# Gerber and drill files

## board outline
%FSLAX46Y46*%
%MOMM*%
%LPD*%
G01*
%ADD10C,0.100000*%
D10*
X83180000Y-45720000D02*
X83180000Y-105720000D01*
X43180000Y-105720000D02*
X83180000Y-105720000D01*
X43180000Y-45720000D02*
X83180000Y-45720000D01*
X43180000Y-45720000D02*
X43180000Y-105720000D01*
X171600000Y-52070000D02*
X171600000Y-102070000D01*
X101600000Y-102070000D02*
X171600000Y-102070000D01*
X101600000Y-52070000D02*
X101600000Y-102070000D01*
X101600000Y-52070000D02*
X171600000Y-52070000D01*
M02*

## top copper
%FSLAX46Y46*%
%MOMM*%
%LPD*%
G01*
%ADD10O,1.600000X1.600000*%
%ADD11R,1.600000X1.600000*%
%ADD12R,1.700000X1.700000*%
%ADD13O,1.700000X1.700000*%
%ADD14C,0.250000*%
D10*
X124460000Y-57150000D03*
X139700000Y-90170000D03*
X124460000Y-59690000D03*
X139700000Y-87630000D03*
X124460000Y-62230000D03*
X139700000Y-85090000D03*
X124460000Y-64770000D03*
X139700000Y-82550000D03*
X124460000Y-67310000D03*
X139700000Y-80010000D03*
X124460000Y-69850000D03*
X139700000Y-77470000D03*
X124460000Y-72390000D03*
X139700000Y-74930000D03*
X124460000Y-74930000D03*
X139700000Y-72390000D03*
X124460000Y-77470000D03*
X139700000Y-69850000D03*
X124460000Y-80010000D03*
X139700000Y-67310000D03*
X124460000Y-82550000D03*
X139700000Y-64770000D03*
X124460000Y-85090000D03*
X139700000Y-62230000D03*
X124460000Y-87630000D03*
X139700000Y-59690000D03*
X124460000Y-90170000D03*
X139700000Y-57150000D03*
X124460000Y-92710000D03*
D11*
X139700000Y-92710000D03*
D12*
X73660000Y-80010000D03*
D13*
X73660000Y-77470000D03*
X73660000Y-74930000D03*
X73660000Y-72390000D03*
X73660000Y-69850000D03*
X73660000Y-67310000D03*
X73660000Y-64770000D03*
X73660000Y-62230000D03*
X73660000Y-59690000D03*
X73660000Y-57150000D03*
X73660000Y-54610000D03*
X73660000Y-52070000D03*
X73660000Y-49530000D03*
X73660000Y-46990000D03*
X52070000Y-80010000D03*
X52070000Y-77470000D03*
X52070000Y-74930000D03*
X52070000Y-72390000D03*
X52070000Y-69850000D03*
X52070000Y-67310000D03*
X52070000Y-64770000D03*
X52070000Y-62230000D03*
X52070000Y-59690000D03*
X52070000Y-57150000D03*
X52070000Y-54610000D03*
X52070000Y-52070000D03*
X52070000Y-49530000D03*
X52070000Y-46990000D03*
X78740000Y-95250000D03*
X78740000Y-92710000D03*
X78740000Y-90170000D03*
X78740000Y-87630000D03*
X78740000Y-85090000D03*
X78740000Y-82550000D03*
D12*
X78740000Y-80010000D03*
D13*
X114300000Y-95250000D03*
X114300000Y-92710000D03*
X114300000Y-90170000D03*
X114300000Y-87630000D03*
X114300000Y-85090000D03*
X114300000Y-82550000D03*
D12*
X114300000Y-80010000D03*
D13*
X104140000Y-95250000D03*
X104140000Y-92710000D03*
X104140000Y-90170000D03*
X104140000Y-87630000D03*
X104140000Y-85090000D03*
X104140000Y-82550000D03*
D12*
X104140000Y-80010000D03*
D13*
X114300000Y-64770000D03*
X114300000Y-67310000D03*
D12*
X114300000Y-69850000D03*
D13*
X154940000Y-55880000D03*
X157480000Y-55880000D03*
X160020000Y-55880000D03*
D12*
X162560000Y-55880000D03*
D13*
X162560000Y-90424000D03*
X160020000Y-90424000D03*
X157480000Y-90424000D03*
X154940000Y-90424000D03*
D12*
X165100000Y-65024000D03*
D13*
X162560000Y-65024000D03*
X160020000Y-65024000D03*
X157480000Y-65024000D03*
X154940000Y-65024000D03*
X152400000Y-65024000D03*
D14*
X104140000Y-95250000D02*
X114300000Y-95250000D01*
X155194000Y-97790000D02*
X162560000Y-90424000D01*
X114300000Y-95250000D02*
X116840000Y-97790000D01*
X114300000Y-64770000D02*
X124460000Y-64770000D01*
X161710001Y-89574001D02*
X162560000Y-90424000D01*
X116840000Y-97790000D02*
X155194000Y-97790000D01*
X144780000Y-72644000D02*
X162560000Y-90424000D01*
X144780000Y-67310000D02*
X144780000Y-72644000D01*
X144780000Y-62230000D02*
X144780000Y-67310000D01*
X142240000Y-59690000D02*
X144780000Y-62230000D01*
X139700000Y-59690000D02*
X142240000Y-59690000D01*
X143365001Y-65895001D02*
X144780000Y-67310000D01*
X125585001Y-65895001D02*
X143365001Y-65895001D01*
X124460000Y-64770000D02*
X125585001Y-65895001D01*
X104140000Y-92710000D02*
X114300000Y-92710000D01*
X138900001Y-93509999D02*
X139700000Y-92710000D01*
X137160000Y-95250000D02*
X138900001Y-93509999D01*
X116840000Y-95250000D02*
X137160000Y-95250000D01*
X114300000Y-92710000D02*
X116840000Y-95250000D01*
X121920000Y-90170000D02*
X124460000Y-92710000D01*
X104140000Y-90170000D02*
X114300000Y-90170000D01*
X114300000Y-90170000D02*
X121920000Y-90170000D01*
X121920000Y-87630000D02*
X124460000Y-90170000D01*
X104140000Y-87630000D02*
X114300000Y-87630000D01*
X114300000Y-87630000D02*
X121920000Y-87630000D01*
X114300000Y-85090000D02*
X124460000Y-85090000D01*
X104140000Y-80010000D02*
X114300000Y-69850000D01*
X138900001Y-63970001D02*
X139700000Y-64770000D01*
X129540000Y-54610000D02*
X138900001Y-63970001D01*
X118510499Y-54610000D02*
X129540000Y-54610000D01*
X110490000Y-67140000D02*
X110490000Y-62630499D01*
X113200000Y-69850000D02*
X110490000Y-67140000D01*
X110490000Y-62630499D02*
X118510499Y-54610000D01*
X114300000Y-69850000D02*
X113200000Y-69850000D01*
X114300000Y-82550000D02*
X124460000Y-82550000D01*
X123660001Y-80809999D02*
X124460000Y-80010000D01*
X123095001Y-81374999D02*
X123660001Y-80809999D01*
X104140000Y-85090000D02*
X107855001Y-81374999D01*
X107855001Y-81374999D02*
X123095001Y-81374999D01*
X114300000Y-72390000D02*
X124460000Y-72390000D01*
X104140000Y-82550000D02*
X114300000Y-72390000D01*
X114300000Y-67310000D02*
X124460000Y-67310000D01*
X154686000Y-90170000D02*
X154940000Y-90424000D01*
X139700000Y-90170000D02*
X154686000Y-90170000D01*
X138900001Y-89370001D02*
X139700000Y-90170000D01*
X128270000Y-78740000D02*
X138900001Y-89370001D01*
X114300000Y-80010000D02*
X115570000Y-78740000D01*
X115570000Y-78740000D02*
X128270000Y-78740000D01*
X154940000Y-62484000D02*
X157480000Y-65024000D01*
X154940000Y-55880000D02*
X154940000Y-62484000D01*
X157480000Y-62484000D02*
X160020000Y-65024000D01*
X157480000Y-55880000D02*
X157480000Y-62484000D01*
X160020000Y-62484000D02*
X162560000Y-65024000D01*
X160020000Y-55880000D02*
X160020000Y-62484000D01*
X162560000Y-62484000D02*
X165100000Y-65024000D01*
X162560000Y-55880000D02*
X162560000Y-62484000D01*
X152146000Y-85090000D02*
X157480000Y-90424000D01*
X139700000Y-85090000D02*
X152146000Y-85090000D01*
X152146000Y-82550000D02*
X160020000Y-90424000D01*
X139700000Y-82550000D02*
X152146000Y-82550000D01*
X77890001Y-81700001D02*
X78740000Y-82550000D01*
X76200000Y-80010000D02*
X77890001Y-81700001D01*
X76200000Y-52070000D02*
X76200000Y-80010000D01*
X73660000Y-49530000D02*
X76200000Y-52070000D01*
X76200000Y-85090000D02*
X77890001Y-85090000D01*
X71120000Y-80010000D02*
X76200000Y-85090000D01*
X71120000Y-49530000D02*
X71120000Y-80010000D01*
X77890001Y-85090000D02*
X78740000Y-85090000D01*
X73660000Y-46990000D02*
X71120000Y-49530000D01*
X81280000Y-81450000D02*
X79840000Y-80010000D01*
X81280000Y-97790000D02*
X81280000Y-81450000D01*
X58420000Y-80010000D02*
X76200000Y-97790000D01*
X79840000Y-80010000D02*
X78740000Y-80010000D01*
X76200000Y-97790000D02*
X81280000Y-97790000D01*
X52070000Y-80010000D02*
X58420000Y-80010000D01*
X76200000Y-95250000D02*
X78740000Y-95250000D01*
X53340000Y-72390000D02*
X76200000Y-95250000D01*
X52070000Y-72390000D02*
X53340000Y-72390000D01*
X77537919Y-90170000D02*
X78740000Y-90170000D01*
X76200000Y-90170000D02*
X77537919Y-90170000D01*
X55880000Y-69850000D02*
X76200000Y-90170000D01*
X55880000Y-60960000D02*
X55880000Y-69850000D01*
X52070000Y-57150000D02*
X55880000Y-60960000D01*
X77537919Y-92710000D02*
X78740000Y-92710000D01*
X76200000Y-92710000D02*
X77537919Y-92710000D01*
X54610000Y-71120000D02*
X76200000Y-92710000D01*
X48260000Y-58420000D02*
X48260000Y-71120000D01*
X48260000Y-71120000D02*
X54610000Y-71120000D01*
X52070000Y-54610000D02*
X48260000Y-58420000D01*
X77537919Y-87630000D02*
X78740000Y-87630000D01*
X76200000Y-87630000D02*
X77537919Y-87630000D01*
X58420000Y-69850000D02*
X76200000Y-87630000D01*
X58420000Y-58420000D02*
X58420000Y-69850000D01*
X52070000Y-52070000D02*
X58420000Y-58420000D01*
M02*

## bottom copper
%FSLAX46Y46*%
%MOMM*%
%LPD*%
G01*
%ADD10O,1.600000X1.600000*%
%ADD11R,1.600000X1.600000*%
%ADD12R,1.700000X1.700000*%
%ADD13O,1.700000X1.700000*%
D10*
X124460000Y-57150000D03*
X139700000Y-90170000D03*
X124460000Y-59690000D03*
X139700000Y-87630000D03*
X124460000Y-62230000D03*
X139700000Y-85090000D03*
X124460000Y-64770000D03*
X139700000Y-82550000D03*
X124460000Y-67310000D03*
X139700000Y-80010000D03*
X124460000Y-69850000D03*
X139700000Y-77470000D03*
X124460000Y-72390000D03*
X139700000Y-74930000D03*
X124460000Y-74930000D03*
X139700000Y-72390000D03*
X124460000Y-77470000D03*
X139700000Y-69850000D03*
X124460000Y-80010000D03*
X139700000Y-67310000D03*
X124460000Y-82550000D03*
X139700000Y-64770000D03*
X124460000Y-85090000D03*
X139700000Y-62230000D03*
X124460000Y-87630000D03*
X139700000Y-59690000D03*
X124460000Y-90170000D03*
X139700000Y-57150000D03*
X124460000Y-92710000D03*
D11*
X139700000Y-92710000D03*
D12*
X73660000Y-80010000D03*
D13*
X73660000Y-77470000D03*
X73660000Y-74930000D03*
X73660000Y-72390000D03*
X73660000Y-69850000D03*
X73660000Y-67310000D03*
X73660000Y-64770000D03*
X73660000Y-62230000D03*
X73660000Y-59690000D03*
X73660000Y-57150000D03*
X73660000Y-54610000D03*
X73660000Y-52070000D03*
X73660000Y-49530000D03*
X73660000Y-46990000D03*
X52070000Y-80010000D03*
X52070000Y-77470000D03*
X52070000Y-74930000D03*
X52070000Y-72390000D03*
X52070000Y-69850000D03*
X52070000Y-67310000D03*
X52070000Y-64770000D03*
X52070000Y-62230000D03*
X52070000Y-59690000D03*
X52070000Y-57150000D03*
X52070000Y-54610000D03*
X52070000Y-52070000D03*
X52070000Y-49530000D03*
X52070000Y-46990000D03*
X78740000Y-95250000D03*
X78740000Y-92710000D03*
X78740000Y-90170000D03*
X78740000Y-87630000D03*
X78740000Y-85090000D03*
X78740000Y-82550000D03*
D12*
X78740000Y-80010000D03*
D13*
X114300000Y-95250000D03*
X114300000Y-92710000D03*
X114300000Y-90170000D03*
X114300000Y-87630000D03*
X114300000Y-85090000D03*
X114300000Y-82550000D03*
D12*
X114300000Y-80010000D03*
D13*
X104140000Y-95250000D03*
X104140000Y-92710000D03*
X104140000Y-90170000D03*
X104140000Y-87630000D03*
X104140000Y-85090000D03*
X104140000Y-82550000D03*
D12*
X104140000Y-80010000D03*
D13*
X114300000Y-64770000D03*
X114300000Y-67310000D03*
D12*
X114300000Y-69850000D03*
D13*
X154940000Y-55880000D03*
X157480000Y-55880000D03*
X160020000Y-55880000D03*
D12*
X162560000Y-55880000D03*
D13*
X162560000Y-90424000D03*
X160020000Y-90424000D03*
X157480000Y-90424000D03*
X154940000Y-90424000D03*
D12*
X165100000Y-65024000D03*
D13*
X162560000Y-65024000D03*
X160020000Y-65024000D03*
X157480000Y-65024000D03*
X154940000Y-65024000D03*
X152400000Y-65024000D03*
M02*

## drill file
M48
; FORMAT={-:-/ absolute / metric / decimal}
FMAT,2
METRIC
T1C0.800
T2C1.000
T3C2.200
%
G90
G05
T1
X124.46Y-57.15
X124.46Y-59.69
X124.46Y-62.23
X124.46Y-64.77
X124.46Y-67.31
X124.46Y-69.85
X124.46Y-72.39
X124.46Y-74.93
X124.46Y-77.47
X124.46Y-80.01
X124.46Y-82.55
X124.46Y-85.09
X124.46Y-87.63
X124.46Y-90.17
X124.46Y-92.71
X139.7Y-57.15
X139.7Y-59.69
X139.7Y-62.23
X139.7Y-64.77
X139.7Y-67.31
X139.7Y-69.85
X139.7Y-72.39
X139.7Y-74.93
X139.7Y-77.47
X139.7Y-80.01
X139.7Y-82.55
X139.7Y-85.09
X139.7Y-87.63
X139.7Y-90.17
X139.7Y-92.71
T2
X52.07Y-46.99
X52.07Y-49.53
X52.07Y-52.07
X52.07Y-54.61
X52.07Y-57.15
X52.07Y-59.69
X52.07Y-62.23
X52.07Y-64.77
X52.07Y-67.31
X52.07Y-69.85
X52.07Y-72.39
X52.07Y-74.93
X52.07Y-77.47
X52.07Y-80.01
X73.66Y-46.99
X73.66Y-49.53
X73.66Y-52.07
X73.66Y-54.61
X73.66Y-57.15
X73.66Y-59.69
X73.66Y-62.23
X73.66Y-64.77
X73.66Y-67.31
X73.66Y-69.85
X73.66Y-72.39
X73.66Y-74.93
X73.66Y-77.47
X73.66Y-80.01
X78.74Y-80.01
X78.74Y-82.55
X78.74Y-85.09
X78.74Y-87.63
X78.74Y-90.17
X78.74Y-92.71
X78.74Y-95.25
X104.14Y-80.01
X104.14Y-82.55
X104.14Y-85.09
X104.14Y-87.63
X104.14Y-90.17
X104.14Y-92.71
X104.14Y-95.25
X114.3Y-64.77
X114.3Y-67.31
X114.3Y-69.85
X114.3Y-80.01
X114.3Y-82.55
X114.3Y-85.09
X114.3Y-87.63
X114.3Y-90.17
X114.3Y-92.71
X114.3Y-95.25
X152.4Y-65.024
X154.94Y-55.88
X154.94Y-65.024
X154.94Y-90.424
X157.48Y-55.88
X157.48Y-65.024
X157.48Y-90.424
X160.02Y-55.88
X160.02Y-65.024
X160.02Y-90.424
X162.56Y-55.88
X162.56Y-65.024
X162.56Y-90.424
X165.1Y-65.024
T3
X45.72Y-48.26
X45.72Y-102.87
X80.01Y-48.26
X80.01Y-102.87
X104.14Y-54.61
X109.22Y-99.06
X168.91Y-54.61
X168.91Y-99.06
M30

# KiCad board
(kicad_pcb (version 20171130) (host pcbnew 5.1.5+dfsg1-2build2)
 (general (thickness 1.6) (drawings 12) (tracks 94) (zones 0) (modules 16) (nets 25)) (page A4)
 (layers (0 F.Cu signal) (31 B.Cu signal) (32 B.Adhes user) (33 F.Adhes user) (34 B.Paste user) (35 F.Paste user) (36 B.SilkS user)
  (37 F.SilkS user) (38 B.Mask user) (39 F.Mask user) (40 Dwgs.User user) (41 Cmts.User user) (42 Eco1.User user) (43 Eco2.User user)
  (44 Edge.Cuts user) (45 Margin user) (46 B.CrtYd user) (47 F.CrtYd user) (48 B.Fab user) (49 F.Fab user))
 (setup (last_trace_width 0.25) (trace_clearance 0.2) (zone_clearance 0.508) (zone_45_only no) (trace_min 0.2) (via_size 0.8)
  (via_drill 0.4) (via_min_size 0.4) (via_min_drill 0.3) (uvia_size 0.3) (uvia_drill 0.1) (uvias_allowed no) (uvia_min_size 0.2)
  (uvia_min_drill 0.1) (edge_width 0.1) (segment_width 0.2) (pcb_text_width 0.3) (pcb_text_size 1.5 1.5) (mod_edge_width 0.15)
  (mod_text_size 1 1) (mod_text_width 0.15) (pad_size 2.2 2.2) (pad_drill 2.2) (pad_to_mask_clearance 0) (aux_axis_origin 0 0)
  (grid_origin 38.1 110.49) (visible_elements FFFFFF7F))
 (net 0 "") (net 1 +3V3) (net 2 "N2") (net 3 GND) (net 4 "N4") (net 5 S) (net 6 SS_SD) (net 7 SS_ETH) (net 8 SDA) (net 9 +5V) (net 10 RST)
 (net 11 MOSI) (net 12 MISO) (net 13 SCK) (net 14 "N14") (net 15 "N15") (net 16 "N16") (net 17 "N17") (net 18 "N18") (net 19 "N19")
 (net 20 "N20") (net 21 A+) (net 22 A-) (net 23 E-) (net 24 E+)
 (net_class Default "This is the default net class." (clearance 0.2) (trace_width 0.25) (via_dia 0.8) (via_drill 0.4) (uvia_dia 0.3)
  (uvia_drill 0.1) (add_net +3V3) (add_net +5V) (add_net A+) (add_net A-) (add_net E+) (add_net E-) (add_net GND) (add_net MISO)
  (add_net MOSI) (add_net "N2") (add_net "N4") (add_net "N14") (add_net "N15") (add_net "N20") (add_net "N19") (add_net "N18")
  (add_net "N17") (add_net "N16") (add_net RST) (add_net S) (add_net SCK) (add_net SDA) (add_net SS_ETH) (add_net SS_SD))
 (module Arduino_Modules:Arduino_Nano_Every (layer F.Cu) (at 139.7 92.71 180)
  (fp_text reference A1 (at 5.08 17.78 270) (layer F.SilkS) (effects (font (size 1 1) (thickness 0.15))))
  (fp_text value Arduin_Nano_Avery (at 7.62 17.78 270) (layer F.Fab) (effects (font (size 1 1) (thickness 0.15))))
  (pad 16 thru_hole oval (at 15.24 35.56) (size 1.6 1.6) (drill 0.8) (layers *.Cu *.Mask))
  (pad 2 thru_hole oval (at 0 2.54) (size 1.6 1.6) (drill 0.8) (layers *.Cu *.Mask) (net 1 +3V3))
  (pad 17 thru_hole oval (at 15.24 33.02) (size 1.6 1.6) (drill 0.8) (layers *.Cu *.Mask))
  (pad 3 thru_hole oval (at 0 5.08) (size 1.6 1.6) (drill 0.8) (layers *.Cu *.Mask))
  (pad 18 thru_hole oval (at 15.24 30.48) (size 1.6 1.6) (drill 0.8) (layers *.Cu *.Mask))
  (pad 4 thru_hole oval (at 0 7.62) (size 1.6 1.6) (drill 0.8) (layers *.Cu *.Mask) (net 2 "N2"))
  (pad 19 thru_hole oval (at 15.24 27.94) (size 1.6 1.6) (drill 0.8) (layers *.Cu *.Mask) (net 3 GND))
  (pad 5 thru_hole oval (at 0 10.16) (size 1.6 1.6) (drill 0.8) (layers *.Cu *.Mask) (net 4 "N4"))
  (pad 20 thru_hole oval (at 15.24 25.4) (size 1.6 1.6) (drill 0.8) (layers *.Cu *.Mask) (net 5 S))
  (pad 6 thru_hole oval (at 0 12.7) (size 1.6 1.6) (drill 0.8) (layers *.Cu *.Mask))
  (pad 21 thru_hole oval (at 15.24 22.86) (size 1.6 1.6) (drill 0.8) (layers *.Cu *.Mask))
  (pad 7 thru_hole oval (at 0 15.24) (size 1.6 1.6) (drill 0.8) (layers *.Cu *.Mask))
  (pad 22 thru_hole oval (at 15.24 20.32) (size 1.6 1.6) (drill 0.8) (layers *.Cu *.Mask) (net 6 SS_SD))
  (pad 8 thru_hole oval (at 0 17.78) (size 1.6 1.6) (drill 0.8) (layers *.Cu *.Mask))
  (pad 23 thru_hole oval (at 15.24 17.78) (size 1.6 1.6) (drill 0.8) (layers *.Cu *.Mask))
  (pad 9 thru_hole oval (at 0 20.32) (size 1.6 1.6) (drill 0.8) (layers *.Cu *.Mask))
  (pad 24 thru_hole oval (at 15.24 15.24) (size 1.6 1.6) (drill 0.8) (layers *.Cu *.Mask))
  (pad 10 thru_hole oval (at 0 22.86) (size 1.6 1.6) (drill 0.8) (layers *.Cu *.Mask))
  (pad 25 thru_hole oval (at 15.24 12.7) (size 1.6 1.6) (drill 0.8) (layers *.Cu *.Mask) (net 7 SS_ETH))
  (pad 11 thru_hole oval (at 0 25.4) (size 1.6 1.6) (drill 0.8) (layers *.Cu *.Mask))
  (pad 26 thru_hole oval (at 15.24 10.16) (size 1.6 1.6) (drill 0.8) (layers *.Cu *.Mask) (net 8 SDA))
  (pad 12 thru_hole oval (at 0 27.94) (size 1.6 1.6) (drill 0.8) (layers *.Cu *.Mask) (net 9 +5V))
  (pad 27 thru_hole oval (at 15.24 7.62) (size 1.6 1.6) (drill 0.8) (layers *.Cu *.Mask) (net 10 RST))
  (pad 13 thru_hole oval (at 0 30.48) (size 1.6 1.6) (drill 0.8) (layers *.Cu *.Mask))
  (pad 28 thru_hole oval (at 15.24 5.08) (size 1.6 1.6) (drill 0.8) (layers *.Cu *.Mask))
  (pad 14 thru_hole oval (at 0 33.02) (size 1.6 1.6) (drill 0.8) (layers *.Cu *.Mask) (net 3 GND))
  (pad 29 thru_hole oval (at 15.24 2.54) (size 1.6 1.6) (drill 0.8) (layers *.Cu *.Mask) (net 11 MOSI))
  (pad 15 thru_hole oval (at 0 35.56) (size 1.6 1.6) (drill 0.8) (layers *.Cu *.Mask))
  (pad 30 thru_hole oval (at 15.24 0) (size 1.6 1.6) (drill 0.8) (layers *.Cu *.Mask) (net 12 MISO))
  (pad 1 thru_hole rect (at 0 0) (size 1.6 1.6) (drill 0.8) (layers *.Cu *.Mask) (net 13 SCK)))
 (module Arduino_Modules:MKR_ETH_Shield (layer F.Cu) (at 73.66 80.01 180)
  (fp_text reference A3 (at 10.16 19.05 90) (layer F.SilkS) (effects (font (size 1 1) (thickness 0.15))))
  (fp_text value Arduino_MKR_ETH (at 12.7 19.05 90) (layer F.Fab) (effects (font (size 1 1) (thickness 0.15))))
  (pad 1 thru_hole rect (at 0 0) (size 1.7 1.7) (drill 1) (layers *.Cu *.Mask))
  (pad 2 thru_hole oval (at 0 2.54) (size 1.7 1.7) (drill 1) (layers *.Cu *.Mask))
  (pad 3 thru_hole oval (at 0 5.08) (size 1.7 1.7) (drill 1) (layers *.Cu *.Mask))
  (pad 4 thru_hole oval (at 0 7.62) (size 1.7 1.7) (drill 1) (layers *.Cu *.Mask))
  (pad 5 thru_hole oval (at 0 10.16) (size 1.7 1.7) (drill 1) (layers *.Cu *.Mask))
  (pad 6 thru_hole oval (at 0 12.7) (size 1.7 1.7) (drill 1) (layers *.Cu *.Mask))
  (pad 7 thru_hole oval (at 0 15.24) (size 1.7 1.7) (drill 1) (layers *.Cu *.Mask))
  (pad 8 thru_hole oval (at 0 17.78) (size 1.7 1.7) (drill 1) (layers *.Cu *.Mask))
  (pad 9 thru_hole oval (at 0 20.32) (size 1.7 1.7) (drill 1) (layers *.Cu *.Mask))
  (pad 10 thru_hole oval (at 0 22.86) (size 1.7 1.7) (drill 1) (layers *.Cu *.Mask))
  (pad 11 thru_hole oval (at 0 25.4) (size 1.7 1.7) (drill 1) (layers *.Cu *.Mask))
  (pad 12 thru_hole oval (at 0 27.94) (size 1.7 1.7) (drill 1) (layers *.Cu *.Mask))
  (pad 13 thru_hole oval (at 0 30.48) (size 1.7 1.7) (drill 1) (layers *.Cu *.Mask) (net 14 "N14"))
  (pad 14 thru_hole oval (at 0 33.02) (size 1.7 1.7) (drill 1) (layers *.Cu *.Mask) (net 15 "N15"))
  (pad 28 thru_hole oval (at 21.59 0) (size 1.7 1.7) (drill 1) (layers *.Cu *.Mask) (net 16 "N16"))
  (pad 27 thru_hole oval (at 21.59 2.54) (size 1.7 1.7) (drill 1) (layers *.Cu *.Mask))
  (pad 26 thru_hole oval (at 21.59 5.08) (size 1.7 1.7) (drill 1) (layers *.Cu *.Mask))
  (pad 25 thru_hole oval (at 21.59 7.62) (size 1.7 1.7) (drill 1) (layers *.Cu *.Mask) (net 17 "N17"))
  (pad 24 thru_hole oval (at 21.59 10.16) (size 1.7 1.7) (drill 1) (layers *.Cu *.Mask))
  (pad 23 thru_hole oval (at 21.59 12.7) (size 1.7 1.7) (drill 1) (layers *.Cu *.Mask))
  (pad 22 thru_hole oval (at 21.59 15.24) (size 1.7 1.7) (drill 1) (layers *.Cu *.Mask))
  (pad 21 thru_hole oval (at 21.59 17.78) (size 1.7 1.7) (drill 1) (layers *.Cu *.Mask))
  (pad 20 thru_hole oval (at 21.59 20.32) (size 1.7 1.7) (drill 1) (layers *.Cu *.Mask))
  (pad 19 thru_hole oval (at 21.59 22.86) (size 1.7 1.7) (drill 1) (layers *.Cu *.Mask) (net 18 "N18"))
  (pad 18 thru_hole oval (at 21.59 25.4) (size 1.7 1.7) (drill 1) (layers *.Cu *.Mask) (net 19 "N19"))
  (pad 17 thru_hole oval (at 21.59 27.94) (size 1.7 1.7) (drill 1) (layers *.Cu *.Mask) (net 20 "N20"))
  (pad 16 thru_hole oval (at 21.59 30.48) (size 1.7 1.7) (drill 1) (layers *.Cu *.Mask))
  (pad 15 thru_hole oval (at 21.59 33.02) (size 1.7 1.7) (drill 1) (layers *.Cu *.Mask)))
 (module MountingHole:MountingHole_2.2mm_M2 (layer F.Cu) (at 80.01 48.26)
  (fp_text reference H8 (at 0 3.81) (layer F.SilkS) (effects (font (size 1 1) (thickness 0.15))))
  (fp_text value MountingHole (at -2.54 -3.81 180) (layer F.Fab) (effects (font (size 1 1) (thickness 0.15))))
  (pad 1 np_thru_hole circle (at 0 0) (size 2.2 2.2) (drill 2.2) (layers *.Cu *.Mask)))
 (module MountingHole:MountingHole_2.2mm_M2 (layer F.Cu) (at 80.01 102.87)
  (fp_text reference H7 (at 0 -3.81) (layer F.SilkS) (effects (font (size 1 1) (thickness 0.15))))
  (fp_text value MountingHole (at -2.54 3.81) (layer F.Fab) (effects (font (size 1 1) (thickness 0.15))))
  (pad 1 np_thru_hole circle (at 0 0) (size 2.2 2.2) (drill 2.2) (layers *.Cu *.Mask)))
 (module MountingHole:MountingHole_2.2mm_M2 (layer F.Cu) (at 45.72 102.87)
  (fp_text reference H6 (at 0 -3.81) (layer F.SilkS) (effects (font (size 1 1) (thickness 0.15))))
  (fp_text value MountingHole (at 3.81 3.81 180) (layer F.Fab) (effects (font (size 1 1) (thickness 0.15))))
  (pad 1 np_thru_hole circle (at 0 0) (size 2.2 2.2) (drill 2.2) (layers *.Cu *.Mask)))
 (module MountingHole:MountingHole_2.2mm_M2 (layer F.Cu) (at 45.72 48.26)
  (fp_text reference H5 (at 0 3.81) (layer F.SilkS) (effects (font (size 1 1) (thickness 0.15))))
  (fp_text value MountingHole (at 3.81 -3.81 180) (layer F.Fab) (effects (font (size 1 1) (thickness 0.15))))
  (pad 1 np_thru_hole circle (at 0 0) (size 2.2 2.2) (drill 2.2) (layers *.Cu *.Mask)))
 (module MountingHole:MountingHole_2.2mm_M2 (layer F.Cu) (at 168.91 54.61)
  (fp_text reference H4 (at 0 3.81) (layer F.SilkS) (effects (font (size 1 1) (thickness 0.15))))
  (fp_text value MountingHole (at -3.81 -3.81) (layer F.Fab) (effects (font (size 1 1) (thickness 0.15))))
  (pad 1 np_thru_hole circle (at 0 0) (size 2.2 2.2) (drill 2.2) (layers *.Cu *.Mask)))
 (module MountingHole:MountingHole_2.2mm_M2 (layer F.Cu) (at 168.91 99.06)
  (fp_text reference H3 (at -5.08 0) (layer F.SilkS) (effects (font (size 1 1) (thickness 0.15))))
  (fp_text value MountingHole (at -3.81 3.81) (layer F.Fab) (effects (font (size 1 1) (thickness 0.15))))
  (pad 1 np_thru_hole circle (at 0 0) (size 2.2 2.2) (drill 2.2) (layers *.Cu *.Mask)))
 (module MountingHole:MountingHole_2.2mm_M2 (layer F.Cu) (at 109.22 99.06)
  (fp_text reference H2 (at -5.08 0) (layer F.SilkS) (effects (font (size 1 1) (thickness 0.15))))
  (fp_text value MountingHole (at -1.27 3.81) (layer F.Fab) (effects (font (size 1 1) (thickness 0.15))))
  (pad 1 np_thru_hole circle (at 0 0) (size 2.2 2.2) (drill 2.2) (layers *.Cu *.Mask)))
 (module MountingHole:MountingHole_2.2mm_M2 (layer F.Cu) (at 104.14 54.61)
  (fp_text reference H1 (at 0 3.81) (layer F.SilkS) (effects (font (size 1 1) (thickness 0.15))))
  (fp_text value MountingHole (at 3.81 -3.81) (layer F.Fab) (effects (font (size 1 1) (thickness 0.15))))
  (pad 1 np_thru_hole circle (at 0 0) (size 2.2 2.2) (drill 2.2) (layers *.Cu *.Mask)))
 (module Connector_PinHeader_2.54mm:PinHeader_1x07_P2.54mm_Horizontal (layer F.Cu) (at 78.74 80.01)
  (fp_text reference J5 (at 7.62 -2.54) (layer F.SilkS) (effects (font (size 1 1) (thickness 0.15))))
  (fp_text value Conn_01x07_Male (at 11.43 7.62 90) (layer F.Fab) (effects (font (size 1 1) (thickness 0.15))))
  (pad 7 thru_hole oval (at 0 15.24) (size 1.7 1.7) (drill 1) (layers *.Cu *.Mask) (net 17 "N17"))
  (pad 6 thru_hole oval (at 0 12.7) (size 1.7 1.7) (drill 1) (layers *.Cu *.Mask) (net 19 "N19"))
  (pad 5 thru_hole oval (at 0 10.16) (size 1.7 1.7) (drill 1) (layers *.Cu *.Mask) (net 18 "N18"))
  (pad 4 thru_hole oval (at 0 7.62) (size 1.7 1.7) (drill 1) (layers *.Cu *.Mask) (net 20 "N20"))
  (pad 3 thru_hole oval (at 0 5.08) (size 1.7 1.7) (drill 1) (layers *.Cu *.Mask) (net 15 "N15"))
  (pad 2 thru_hole oval (at 0 2.54) (size 1.7 1.7) (drill 1) (layers *.Cu *.Mask) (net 14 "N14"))
  (pad 1 thru_hole rect (at 0 0) (size 1.7 1.7) (drill 1) (layers *.Cu *.Mask) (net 16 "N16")))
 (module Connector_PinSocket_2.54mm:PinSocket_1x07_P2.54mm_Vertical (layer F.Cu) (at 114.3 80.01)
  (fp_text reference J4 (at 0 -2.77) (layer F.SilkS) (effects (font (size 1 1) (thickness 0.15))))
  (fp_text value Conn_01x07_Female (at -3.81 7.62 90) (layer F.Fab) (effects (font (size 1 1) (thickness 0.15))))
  (pad 7 thru_hole oval (at 0 15.24) (size 1.7 1.7) (drill 1) (layers *.Cu *.Mask) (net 3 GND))
  (pad 6 thru_hole oval (at 0 12.7) (size 1.7 1.7) (drill 1) (layers *.Cu *.Mask) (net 13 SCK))
  (pad 5 thru_hole oval (at 0 10.16) (size 1.7 1.7) (drill 1) (layers *.Cu *.Mask) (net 12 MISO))
  (pad 4 thru_hole oval (at 0 7.62) (size 1.7 1.7) (drill 1) (layers *.Cu *.Mask) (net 11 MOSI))
  (pad 3 thru_hole oval (at 0 5.08) (size 1.7 1.7) (drill 1) (layers *.Cu *.Mask) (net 10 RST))
  (pad 2 thru_hole oval (at 0 2.54) (size 1.7 1.7) (drill 1) (layers *.Cu *.Mask) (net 8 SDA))
  (pad 1 thru_hole rect (at 0 0) (size 1.7 1.7) (drill 1) (layers *.Cu *.Mask) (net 1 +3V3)))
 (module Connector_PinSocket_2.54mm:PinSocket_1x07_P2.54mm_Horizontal (layer F.Cu) (at 104.14 80.01)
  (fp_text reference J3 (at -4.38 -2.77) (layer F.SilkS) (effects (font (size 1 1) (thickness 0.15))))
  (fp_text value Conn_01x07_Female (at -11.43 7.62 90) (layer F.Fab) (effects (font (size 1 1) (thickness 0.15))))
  (pad 7 thru_hole oval (at 0 15.24) (size 1.7 1.7) (drill 1) (layers *.Cu *.Mask) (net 3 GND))
  (pad 6 thru_hole oval (at 0 12.7) (size 1.7 1.7) (drill 1) (layers *.Cu *.Mask) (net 13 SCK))
  (pad 5 thru_hole oval (at 0 10.16) (size 1.7 1.7) (drill 1) (layers *.Cu *.Mask) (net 12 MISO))
  (pad 4 thru_hole oval (at 0 7.62) (size 1.7 1.7) (drill 1) (layers *.Cu *.Mask) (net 11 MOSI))
  (pad 3 thru_hole oval (at 0 5.08) (size 1.7 1.7) (drill 1) (layers *.Cu *.Mask) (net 7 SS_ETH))
  (pad 2 thru_hole oval (at 0 2.54) (size 1.7 1.7) (drill 1) (layers *.Cu *.Mask) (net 6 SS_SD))
  (pad 1 thru_hole rect (at 0 0) (size 1.7 1.7) (drill 1) (layers *.Cu *.Mask) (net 9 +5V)))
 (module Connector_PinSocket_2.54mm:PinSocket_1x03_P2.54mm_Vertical (layer F.Cu) (at 114.3 69.85 180)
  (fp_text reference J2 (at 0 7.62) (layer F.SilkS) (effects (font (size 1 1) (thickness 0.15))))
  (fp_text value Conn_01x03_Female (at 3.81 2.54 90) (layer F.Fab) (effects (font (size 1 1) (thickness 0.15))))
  (pad 3 thru_hole oval (at 0 5.08 180) (size 1.7 1.7) (drill 1) (layers *.Cu *.Mask) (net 3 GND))
  (pad 2 thru_hole oval (at 0 2.54 180) (size 1.7 1.7) (drill 1) (layers *.Cu *.Mask) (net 5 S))
  (pad 1 thru_hole rect (at 0 0 180) (size 1.7 1.7) (drill 1) (layers *.Cu *.Mask) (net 9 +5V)))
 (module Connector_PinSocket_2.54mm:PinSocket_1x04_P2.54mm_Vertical (layer F.Cu) (at 162.56 55.88 270)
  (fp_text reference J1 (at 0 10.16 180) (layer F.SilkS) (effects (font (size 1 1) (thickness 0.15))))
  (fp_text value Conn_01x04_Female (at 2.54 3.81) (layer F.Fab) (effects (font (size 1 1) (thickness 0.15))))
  (pad 4 thru_hole oval (at 0 7.62 270) (size 1.7 1.7) (drill 1) (layers *.Cu *.Mask) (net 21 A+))
  (pad 3 thru_hole oval (at 0 5.08 270) (size 1.7 1.7) (drill 1) (layers *.Cu *.Mask) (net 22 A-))
  (pad 2 thru_hole oval (at 0 2.54 270) (size 1.7 1.7) (drill 1) (layers *.Cu *.Mask) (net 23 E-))
  (pad 1 thru_hole rect (at 0 0 270) (size 1.7 1.7) (drill 1) (layers *.Cu *.Mask) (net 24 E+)))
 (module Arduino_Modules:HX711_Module (layer F.Cu) (at 152.4 65.024)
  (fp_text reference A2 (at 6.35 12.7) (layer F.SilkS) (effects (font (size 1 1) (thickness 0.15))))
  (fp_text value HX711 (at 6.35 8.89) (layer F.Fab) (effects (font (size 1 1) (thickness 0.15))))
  (pad 10 thru_hole oval (at 10.16 25.4) (size 1.7 1.7) (drill 1) (layers *.Cu *.Mask) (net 3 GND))
  (pad 9 thru_hole oval (at 7.62 25.4) (size 1.7 1.7) (drill 1) (layers *.Cu *.Mask) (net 4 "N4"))
  (pad 8 thru_hole oval (at 5.08 25.4) (size 1.7 1.7) (drill 1) (layers *.Cu *.Mask) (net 2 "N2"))
  (pad 7 thru_hole oval (at 2.54 25.4) (size 1.7 1.7) (drill 1) (layers *.Cu *.Mask) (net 1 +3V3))
  (pad 1 thru_hole rect (at 12.7 0) (size 1.7 1.7) (drill 1) (layers *.Cu *.Mask) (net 24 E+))
  (pad 2 thru_hole oval (at 10.16 0) (size 1.7 1.7) (drill 1) (layers *.Cu *.Mask) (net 23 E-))
  (pad 3 thru_hole oval (at 7.62 0) (size 1.7 1.7) (drill 1) (layers *.Cu *.Mask) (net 22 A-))
  (pad 4 thru_hole oval (at 5.08 0) (size 1.7 1.7) (drill 1) (layers *.Cu *.Mask) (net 21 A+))
  (pad 5 thru_hole oval (at 2.54 0) (size 1.7 1.7) (drill 1) (layers *.Cu *.Mask))
  (pad 6 thru_hole oval (at 0 0) (size 1.7 1.7) (drill 1) (layers *.Cu *.Mask)))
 (gr_line (start 83.18 45.72) (end 83.18 105.72) (layer Edge.Cuts) (width 0.1))
 (gr_line (start 43.18 105.72) (end 83.18 105.72) (layer Edge.Cuts) (width 0.1))
 (gr_line (start 43.18 45.72) (end 83.18 45.72) (layer Edge.Cuts) (width 0.1))
 (gr_line (start 43.18 45.72) (end 43.18 105.72) (layer Edge.Cuts) (width 0.1))
 (gr_line (start 171.6 52.07) (end 171.6 102.07) (layer Edge.Cuts) (width 0.1))
 (gr_line (start 101.6 102.07) (end 171.6 102.07) (layer Edge.Cuts) (width 0.1))
 (gr_line (start 101.6 52.07) (end 101.6 102.07) (layer Edge.Cuts) (width 0.1))
 (gr_line (start 101.6 52.07) (end 171.6 52.07) (layer Edge.Cuts) (width 0.1))
 (segment (start 104.14 95.25) (end 114.3 95.25) (width 0.25) (layer F.Cu) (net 3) (status 30))
 (segment (start 155.194 97.79) (end 162.56 90.424) (width 0.25) (layer F.Cu) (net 3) (status 20))
 (segment (start 114.3 95.25) (end 116.84 97.79) (width 0.25) (layer F.Cu) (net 3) (status 10))
 (segment (start 114.3 64.77) (end 124.46 64.77) (width 0.25) (layer F.Cu) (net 3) (status 30))
 (segment (start 161.710001 89.574001) (end 162.56 90.424) (width 0.25) (layer F.Cu) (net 3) (status 20))
 (segment (start 116.84 97.79) (end 155.194 97.79) (width 0.25) (layer F.Cu) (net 3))
 (segment (start 144.78 72.644) (end 162.56 90.424) (width 0.25) (layer F.Cu) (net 3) (status 20))
 (segment (start 144.78 67.31) (end 144.78 72.644) (width 0.25) (layer F.Cu) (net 3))
 (segment (start 144.78 62.23) (end 144.78 67.31) (width 0.25) (layer F.Cu) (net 3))
 (segment (start 142.24 59.69) (end 144.78 62.23) (width 0.25) (layer F.Cu) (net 3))
 (segment (start 139.7 59.69) (end 142.24 59.69) (width 0.25) (layer F.Cu) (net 3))
 (segment (start 143.365001 65.895001) (end 144.78 67.31) (width 0.25) (layer F.Cu) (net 3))
 (segment (start 125.585001 65.895001) (end 143.365001 65.895001) (width 0.25) (layer F.Cu) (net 3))
 (segment (start 124.46 64.77) (end 125.585001 65.895001) (width 0.25) (layer F.Cu) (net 3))
 (segment (start 104.14 92.71) (end 114.3 92.71) (width 0.25) (layer F.Cu) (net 13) (status 30))
 (segment (start 138.900001 93.509999) (end 139.7 92.71) (width 0.25) (layer F.Cu) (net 13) (status 30))
 (segment (start 137.16 95.25) (end 138.900001 93.509999) (width 0.25) (layer F.Cu) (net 13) (status 20))
 (segment (start 116.84 95.25) (end 137.16 95.25) (width 0.25) (layer F.Cu) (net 13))
 (segment (start 114.3 92.71) (end 116.84 95.25) (width 0.25) (layer F.Cu) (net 13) (status 10))
 (segment (start 121.92 90.17) (end 124.46 92.71) (width 0.25) (layer F.Cu) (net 12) (status 20))
 (segment (start 104.14 90.17) (end 114.3 90.17) (width 0.25) (layer F.Cu) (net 12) (status 30))
 (segment (start 114.3 90.17) (end 121.92 90.17) (width 0.25) (layer F.Cu) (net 12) (status 10))
 (segment (start 121.92 87.63) (end 124.46 90.17) (width 0.25) (layer F.Cu) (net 11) (status 20))
 (segment (start 104.14 87.63) (end 114.3 87.63) (width 0.25) (layer F.Cu) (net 11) (status 30))
 (segment (start 114.3 87.63) (end 121.92 87.63) (width 0.25) (layer F.Cu) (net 11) (status 10))
 (segment (start 114.3 85.09) (end 124.46 85.09) (width 0.25) (layer F.Cu) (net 10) (status 30))
 (segment (start 104.14 80.01) (end 114.3 69.85) (width 0.25) (layer F.Cu) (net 9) (status 30))
 (segment (start 138.900001 63.970001) (end 139.7 64.77) (width 0.25) (layer F.Cu) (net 9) (status 20))
 (segment (start 129.54 54.61) (end 138.900001 63.970001) (width 0.25) (layer F.Cu) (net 9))
 (segment (start 118.510499 54.61) (end 129.54 54.61) (width 0.25) (layer F.Cu) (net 9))
 (segment (start 110.49 67.14) (end 110.49 62.630499) (width 0.25) (layer F.Cu) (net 9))
 (segment (start 113.2 69.85) (end 110.49 67.14) (width 0.25) (layer F.Cu) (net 9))
 (segment (start 110.49 62.630499) (end 118.510499 54.61) (width 0.25) (layer F.Cu) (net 9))
 (segment (start 114.3 69.85) (end 113.2 69.85) (width 0.25) (layer F.Cu) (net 9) (status 10))
 (segment (start 114.3 82.55) (end 124.46 82.55) (width 0.25) (layer F.Cu) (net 8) (status 30))
 (segment (start 123.660001 80.809999) (end 124.46 80.01) (width 0.25) (layer F.Cu) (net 7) (status 20))
 (segment (start 123.095001 81.374999) (end 123.660001 80.809999) (width 0.25) (layer F.Cu) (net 7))
 (segment (start 104.14 85.09) (end 107.855001 81.374999) (width 0.25) (layer F.Cu) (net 7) (status 10))
 (segment (start 107.855001 81.374999) (end 123.095001 81.374999) (width 0.25) (layer F.Cu) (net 7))
 (segment (start 114.3 72.39) (end 124.46 72.39) (width 0.25) (layer F.Cu) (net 6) (status 20))
 (segment (start 104.14 82.55) (end 114.3 72.39) (width 0.25) (layer F.Cu) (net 6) (status 10))
 (segment (start 114.3 67.31) (end 124.46 67.31) (width 0.25) (layer F.Cu) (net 5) (status 30))
 (segment (start 154.686 90.17) (end 154.94 90.424) (width 0.25) (layer F.Cu) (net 1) (status 30))
 (segment (start 139.7 90.17) (end 154.686 90.17) (width 0.25) (layer F.Cu) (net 1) (status 30))
 (segment (start 138.900001 89.370001) (end 139.7 90.17) (width 0.25) (layer F.Cu) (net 1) (status 20))
 (segment (start 128.27 78.74) (end 138.900001 89.370001) (width 0.25) (layer F.Cu) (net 1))
 (segment (start 114.3 80.01) (end 115.57 78.74) (width 0.25) (layer F.Cu) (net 1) (status 10))
 (segment (start 115.57 78.74) (end 128.27 78.74) (width 0.25) (layer F.Cu) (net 1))
 (segment (start 154.94 62.484) (end 157.48 65.024) (width 0.25) (layer F.Cu) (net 21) (status 20))
 (segment (start 154.94 55.88) (end 154.94 62.484) (width 0.25) (layer F.Cu) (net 21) (status 10))
 (segment (start 157.48 62.484) (end 160.02 65.024) (width 0.25) (layer F.Cu) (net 22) (status 20))
 (segment (start 157.48 55.88) (end 157.48 62.484) (width 0.25) (layer F.Cu) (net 22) (status 10))
 (segment (start 160.02 62.484) (end 162.56 65.024) (width 0.25) (layer F.Cu) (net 23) (status 20))
 (segment (start 160.02 55.88) (end 160.02 62.484) (width 0.25) (layer F.Cu) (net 23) (status 10))
 (segment (start 162.56 62.484) (end 165.1 65.024) (width 0.25) (layer F.Cu) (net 24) (status 20))
 (segment (start 162.56 55.88) (end 162.56 62.484) (width 0.25) (layer F.Cu) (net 24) (status 10))
 (segment (start 152.146 85.09) (end 157.48 90.424) (width 0.25) (layer F.Cu) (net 2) (status 20))
 (segment (start 139.7 85.09) (end 152.146 85.09) (width 0.25) (layer F.Cu) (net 2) (status 10))
 (segment (start 152.146 82.55) (end 160.02 90.424) (width 0.25) (layer F.Cu) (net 4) (status 20))
 (segment (start 139.7 82.55) (end 152.146 82.55) (width 0.25) (layer F.Cu) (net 4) (status 10))
 (segment (start 77.890001 81.700001) (end 78.74 82.55) (width 0.25) (layer F.Cu) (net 14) (status 20))
 (segment (start 76.2 80.01) (end 77.890001 81.700001) (width 0.25) (layer F.Cu) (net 14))
 (segment (start 76.2 52.07) (end 76.2 80.01) (width 0.25) (layer F.Cu) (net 14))
 (segment (start 73.66 49.53) (end 76.2 52.07) (width 0.25) (layer F.Cu) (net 14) (status 10))
 (segment (start 76.2 85.09) (end 77.890001 85.09) (width 0.25) (layer F.Cu) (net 15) (status 20))
 (segment (start 71.12 80.01) (end 76.2 85.09) (width 0.25) (layer F.Cu) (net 15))
 (segment (start 71.12 49.53) (end 71.12 80.01) (width 0.25) (layer F.Cu) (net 15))
 (segment (start 77.890001 85.09) (end 78.74 85.09) (width 0.25) (layer F.Cu) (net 15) (status 30))
 (segment (start 73.66 46.99) (end 71.12 49.53) (width 0.25) (layer F.Cu) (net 15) (status 10))
 (segment (start 81.28 81.45) (end 79.84 80.01) (width 0.25) (layer F.Cu) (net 16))
 (segment (start 81.28 97.79) (end 81.28 81.45) (width 0.25) (layer F.Cu) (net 16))
 (segment (start 58.42 80.01) (end 76.2 97.79) (width 0.25) (layer F.Cu) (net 16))
 (segment (start 79.84 80.01) (end 78.74 80.01) (width 0.25) (layer F.Cu) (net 16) (status 20))
 (segment (start 76.2 97.79) (end 81.28 97.79) (width 0.25) (layer F.Cu) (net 16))
 (segment (start 52.07 80.01) (end 58.42 80.01) (width 0.25) (layer F.Cu) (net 16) (status 10))
 (segment (start 76.2 95.25) (end 78.74 95.25) (width 0.25) (layer F.Cu) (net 17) (status 20))
 (segment (start 53.34 72.39) (end 76.2 95.25) (width 0.25) (layer F.Cu) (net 17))
 (segment (start 52.07 72.39) (end 53.34 72.39) (width 0.25) (layer F.Cu) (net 17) (status 10))
 (segment (start 77.537919 90.17) (end 78.74 90.17) (width 0.25) (layer F.Cu) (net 18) (status 20))
 (segment (start 76.2 90.17) (end 77.537919 90.17) (width 0.25) (layer F.Cu) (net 18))
 (segment (start 55.88 69.85) (end 76.2 90.17) (width 0.25) (layer F.Cu) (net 18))
 (segment (start 55.88 60.96) (end 55.88 69.85) (width 0.25) (layer F.Cu) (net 18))
 (segment (start 52.07 57.15) (end 55.88 60.96) (width 0.25) (layer F.Cu) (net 18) (status 10))
 (segment (start 77.537919 92.71) (end 78.74 92.71) (width 0.25) (layer F.Cu) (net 19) (status 20))
 (segment (start 76.2 92.71) (end 77.537919 92.71) (width 0.25) (layer F.Cu) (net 19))
 (segment (start 54.61 71.12) (end 76.2 92.71) (width 0.25) (layer F.Cu) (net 19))
 (segment (start 48.26 58.42) (end 48.26 71.12) (width 0.25) (layer F.Cu) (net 19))
 (segment (start 48.26 71.12) (end 54.61 71.12) (width 0.25) (layer F.Cu) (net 19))
 (segment (start 52.07 54.61) (end 48.26 58.42) (width 0.25) (layer F.Cu) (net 19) (status 10))
 (segment (start 77.537919 87.63) (end 78.74 87.63) (width 0.25) (layer F.Cu) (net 20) (status 20))
 (segment (start 76.2 87.63) (end 77.537919 87.63) (width 0.25) (layer F.Cu) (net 20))
 (segment (start 58.42 69.85) (end 76.2 87.63) (width 0.25) (layer F.Cu) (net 20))
 (segment (start 58.42 58.42) (end 58.42 69.85) (width 0.25) (layer F.Cu) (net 20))
 (segment (start 52.07 52.07) (end 58.42 58.42) (width 0.25) (layer F.Cu) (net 20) (status 10)))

